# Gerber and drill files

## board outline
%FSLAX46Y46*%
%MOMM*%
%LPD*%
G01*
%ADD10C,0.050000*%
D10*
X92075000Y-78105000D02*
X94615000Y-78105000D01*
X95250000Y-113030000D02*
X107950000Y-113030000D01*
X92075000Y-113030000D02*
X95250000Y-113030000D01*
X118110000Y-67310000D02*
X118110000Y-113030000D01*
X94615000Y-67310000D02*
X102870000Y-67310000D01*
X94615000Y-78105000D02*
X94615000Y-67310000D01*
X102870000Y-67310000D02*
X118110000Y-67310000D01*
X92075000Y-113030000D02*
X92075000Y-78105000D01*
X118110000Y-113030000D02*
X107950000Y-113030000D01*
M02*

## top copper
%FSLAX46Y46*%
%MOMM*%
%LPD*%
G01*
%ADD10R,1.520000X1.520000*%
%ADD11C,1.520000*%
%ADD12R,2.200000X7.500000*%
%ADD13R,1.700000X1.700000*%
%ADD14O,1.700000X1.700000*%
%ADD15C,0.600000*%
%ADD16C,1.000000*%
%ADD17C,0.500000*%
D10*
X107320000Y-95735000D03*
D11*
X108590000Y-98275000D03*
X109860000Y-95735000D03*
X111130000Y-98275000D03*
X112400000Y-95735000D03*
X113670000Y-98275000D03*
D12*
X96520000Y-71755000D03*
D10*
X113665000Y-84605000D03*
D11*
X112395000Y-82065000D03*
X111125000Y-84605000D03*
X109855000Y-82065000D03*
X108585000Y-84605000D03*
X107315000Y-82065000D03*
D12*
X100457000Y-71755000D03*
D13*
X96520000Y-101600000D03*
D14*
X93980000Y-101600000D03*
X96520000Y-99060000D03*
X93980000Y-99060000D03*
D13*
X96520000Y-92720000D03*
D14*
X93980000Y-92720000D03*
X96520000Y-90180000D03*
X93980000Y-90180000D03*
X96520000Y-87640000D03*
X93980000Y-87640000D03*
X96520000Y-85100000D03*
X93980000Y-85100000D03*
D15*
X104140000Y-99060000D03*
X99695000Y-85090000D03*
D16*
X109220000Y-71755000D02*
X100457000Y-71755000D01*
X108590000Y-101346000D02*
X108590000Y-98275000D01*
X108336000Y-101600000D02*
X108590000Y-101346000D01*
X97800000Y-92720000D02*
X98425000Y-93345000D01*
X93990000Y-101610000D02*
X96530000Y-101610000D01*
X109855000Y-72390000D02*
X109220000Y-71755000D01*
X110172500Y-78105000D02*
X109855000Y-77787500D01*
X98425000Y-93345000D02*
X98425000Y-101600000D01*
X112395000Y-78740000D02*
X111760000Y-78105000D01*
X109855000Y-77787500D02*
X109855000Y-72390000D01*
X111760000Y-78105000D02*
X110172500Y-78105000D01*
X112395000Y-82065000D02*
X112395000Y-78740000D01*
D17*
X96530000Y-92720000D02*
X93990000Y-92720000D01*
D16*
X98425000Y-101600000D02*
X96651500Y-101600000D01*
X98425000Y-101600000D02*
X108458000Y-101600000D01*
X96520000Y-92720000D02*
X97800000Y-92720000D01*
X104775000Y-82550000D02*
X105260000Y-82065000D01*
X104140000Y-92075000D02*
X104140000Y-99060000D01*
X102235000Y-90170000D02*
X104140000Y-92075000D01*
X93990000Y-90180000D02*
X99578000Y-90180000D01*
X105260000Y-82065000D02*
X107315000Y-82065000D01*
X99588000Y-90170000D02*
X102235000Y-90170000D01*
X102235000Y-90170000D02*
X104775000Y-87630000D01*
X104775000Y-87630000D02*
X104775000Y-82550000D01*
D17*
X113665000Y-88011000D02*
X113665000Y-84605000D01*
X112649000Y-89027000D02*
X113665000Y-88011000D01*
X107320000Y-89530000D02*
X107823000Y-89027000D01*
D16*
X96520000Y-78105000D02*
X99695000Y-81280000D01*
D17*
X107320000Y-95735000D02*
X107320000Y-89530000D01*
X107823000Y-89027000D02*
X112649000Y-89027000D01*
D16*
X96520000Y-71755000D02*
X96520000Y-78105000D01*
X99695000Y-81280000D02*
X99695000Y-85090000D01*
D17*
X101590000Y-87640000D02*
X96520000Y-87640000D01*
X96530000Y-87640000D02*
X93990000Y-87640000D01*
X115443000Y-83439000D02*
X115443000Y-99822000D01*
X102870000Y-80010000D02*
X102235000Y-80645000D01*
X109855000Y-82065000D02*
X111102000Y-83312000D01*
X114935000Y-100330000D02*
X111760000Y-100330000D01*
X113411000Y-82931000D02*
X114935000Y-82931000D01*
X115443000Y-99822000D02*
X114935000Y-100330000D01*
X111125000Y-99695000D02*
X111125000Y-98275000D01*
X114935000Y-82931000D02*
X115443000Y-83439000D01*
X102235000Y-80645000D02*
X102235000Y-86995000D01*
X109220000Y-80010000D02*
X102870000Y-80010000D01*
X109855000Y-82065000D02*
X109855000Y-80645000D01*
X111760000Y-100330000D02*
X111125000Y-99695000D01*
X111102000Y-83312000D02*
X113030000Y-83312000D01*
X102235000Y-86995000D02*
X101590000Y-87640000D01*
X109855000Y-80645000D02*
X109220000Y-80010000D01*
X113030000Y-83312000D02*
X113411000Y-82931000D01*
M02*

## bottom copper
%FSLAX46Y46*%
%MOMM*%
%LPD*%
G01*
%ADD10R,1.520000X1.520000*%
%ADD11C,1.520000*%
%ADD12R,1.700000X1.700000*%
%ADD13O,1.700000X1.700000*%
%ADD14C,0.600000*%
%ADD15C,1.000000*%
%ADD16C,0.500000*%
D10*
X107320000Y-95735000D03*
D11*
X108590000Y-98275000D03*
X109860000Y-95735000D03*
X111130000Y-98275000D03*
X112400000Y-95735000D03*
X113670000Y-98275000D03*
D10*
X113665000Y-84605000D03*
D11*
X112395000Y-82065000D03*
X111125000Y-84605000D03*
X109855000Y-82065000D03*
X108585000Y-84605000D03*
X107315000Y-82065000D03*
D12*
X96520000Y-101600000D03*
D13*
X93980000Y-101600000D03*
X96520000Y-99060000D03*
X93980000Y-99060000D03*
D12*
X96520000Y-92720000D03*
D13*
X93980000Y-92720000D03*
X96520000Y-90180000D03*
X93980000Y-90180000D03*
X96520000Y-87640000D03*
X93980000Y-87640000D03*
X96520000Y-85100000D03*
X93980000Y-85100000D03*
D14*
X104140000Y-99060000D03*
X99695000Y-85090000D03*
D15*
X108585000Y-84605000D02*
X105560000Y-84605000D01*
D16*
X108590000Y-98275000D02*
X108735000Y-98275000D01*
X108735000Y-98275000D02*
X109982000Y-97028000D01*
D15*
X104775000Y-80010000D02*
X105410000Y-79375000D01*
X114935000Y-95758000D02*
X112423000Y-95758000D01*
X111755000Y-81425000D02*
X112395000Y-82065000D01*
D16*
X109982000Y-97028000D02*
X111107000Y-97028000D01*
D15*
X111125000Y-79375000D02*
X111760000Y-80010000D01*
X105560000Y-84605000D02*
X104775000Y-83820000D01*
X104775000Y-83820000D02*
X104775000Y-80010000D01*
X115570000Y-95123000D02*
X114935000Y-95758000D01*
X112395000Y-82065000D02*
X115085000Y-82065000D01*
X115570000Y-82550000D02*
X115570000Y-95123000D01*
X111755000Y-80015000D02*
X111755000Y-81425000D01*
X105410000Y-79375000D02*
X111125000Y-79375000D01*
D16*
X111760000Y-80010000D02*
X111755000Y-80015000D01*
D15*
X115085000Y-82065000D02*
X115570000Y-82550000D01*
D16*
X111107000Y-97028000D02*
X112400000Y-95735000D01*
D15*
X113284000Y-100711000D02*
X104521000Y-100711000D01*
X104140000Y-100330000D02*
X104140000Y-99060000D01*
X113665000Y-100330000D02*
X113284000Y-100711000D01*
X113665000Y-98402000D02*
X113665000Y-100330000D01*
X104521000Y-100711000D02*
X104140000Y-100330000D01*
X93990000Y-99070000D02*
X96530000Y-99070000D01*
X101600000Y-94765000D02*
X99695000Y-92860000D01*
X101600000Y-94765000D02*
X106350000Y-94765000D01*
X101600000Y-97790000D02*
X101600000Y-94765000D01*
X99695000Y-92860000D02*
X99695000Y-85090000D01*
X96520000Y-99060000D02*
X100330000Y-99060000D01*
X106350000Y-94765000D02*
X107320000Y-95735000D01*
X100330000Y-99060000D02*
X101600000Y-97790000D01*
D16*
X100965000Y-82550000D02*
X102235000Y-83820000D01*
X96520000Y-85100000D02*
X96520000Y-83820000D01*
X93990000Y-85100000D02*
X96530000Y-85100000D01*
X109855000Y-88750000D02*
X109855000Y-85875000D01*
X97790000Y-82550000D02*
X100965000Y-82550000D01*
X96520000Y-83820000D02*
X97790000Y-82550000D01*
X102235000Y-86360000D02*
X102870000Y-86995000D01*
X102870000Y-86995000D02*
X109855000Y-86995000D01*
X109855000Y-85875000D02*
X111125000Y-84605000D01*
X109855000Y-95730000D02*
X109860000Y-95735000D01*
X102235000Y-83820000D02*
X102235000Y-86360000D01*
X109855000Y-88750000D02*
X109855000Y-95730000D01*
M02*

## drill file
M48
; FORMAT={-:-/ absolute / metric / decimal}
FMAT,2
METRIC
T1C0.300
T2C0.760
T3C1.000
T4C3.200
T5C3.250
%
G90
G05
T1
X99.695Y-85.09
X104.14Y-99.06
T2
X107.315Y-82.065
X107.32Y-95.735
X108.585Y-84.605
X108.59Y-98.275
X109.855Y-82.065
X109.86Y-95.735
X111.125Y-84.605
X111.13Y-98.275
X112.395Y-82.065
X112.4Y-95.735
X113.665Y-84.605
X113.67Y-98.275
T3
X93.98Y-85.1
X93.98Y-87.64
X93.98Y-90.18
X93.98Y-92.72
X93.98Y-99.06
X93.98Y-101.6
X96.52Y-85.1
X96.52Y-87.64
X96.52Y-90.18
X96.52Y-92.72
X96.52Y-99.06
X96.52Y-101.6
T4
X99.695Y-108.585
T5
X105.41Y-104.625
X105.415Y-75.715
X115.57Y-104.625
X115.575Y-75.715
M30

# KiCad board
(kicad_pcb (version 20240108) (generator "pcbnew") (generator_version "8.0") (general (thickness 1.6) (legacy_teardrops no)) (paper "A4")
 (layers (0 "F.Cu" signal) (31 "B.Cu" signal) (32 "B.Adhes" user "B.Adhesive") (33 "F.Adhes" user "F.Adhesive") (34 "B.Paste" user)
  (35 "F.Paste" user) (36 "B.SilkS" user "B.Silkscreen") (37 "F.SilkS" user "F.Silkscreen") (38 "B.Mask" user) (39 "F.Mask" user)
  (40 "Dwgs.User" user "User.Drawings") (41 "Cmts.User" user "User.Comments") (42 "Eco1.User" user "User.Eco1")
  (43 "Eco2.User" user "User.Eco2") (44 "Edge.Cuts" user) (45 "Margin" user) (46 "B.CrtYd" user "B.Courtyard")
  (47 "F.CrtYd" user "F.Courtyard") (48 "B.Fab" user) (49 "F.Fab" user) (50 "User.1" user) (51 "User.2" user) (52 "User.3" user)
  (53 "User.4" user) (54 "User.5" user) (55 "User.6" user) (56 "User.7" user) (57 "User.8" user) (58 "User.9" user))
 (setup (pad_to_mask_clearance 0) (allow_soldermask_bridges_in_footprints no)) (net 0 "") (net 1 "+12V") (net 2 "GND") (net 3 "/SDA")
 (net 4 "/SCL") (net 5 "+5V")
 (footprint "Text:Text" (layer "F.Cu") (at 106.68 116.84)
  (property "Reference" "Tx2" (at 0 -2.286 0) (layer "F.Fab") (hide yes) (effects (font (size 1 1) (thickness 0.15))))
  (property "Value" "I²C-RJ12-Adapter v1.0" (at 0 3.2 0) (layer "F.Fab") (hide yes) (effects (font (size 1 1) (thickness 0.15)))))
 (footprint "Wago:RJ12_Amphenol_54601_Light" (layer "F.Cu") (at 107.32 95.735)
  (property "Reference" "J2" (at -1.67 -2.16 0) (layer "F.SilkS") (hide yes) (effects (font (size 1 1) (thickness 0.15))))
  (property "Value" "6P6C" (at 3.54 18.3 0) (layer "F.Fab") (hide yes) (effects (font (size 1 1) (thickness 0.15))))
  (pad "" np_thru_hole circle (at -1.91 8.89) (size 3.25 3.25) (drill 3.25) (layers "*.Cu" "*.Mask"))
  (pad "" np_thru_hole circle (at 8.25 8.89) (size 3.25 3.25) (drill 3.25) (layers "*.Cu" "*.Mask"))
  (pad "1" thru_hole rect (at 0 0) (size 1.52 1.52) (drill 0.76) (layers "*.Cu" "*.Mask") (remove_unused_layers no) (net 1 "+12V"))
  (pad "2" thru_hole circle (at 1.27 2.54) (size 1.52 1.52) (drill 0.76) (layers "*.Cu" "*.Mask") (remove_unused_layers no) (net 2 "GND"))
  (pad "3" thru_hole circle (at 2.54 0) (size 1.52 1.52) (drill 0.76) (layers "*.Cu" "*.Mask") (remove_unused_layers no) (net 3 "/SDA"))
  (pad "4" thru_hole circle (at 3.81 2.54) (size 1.52 1.52) (drill 0.76) (layers "*.Cu" "*.Mask") (remove_unused_layers no) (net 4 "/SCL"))
  (pad "5" thru_hole circle (at 5.08 0) (size 1.52 1.52) (drill 0.76) (layers "*.Cu" "*.Mask") (remove_unused_layers no) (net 2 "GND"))
  (pad "6" thru_hole circle (at 6.35 2.54) (size 1.52 1.52) (drill 0.76) (layers "*.Cu" "*.Mask") (remove_unused_layers no) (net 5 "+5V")))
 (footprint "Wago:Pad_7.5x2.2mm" (layer "F.Cu") (at 96.52 71.755 90)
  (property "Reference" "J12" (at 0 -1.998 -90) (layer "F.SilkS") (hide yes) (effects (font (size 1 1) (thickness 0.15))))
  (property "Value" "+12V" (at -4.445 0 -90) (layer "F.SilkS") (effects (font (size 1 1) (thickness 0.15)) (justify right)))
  (pad "1" smd rect (at 0 0 90) (size 7.5 2.2) (layers "F.Cu" "F.Mask") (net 1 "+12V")))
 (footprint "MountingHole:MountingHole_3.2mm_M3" (layer "F.Cu") (at 99.695 108.585)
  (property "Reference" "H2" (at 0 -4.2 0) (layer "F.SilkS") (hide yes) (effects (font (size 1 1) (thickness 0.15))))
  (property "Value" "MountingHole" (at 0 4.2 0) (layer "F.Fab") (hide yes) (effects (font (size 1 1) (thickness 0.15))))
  (pad "" np_thru_hole circle (at 0 0) (size 3.2 3.2) (drill 3.2) (layers "F&B.Cu" "*.Mask")))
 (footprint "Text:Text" (layer "F.Cu") (at 81.28 95.25 90)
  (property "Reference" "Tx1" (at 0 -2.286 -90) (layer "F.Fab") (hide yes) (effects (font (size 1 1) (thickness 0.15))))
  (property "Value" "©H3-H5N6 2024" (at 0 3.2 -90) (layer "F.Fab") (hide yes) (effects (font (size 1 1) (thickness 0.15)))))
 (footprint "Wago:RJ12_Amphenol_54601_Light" (layer "F.Cu") (at 113.665 84.605 180)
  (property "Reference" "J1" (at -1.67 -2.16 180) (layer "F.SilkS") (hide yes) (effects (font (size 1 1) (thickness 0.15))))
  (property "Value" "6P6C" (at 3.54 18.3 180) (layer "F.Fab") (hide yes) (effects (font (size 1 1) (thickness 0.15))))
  (pad "" np_thru_hole circle (at -1.91 8.89 180) (size 3.25 3.25) (drill 3.25) (layers "*.Cu" "*.Mask"))
  (pad "" np_thru_hole circle (at 8.25 8.89 180) (size 3.25 3.25) (drill 3.25) (layers "*.Cu" "*.Mask"))
  (pad "1" thru_hole rect (at 0 0 180) (size 1.52 1.52) (drill 0.76) (layers "*.Cu" "*.Mask") (remove_unused_layers no) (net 1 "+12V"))
  (pad "2" thru_hole circle (at 1.27 2.54 180) (size 1.52 1.52) (drill 0.76) (layers "*.Cu" "*.Mask") (remove_unused_layers no)
   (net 2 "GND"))
  (pad "3" thru_hole circle (at 2.54 0 180) (size 1.52 1.52) (drill 0.76) (layers "*.Cu" "*.Mask") (remove_unused_layers no) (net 3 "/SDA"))
  (pad "4" thru_hole circle (at 3.81 2.54 180) (size 1.52 1.52) (drill 0.76) (layers "*.Cu" "*.Mask") (remove_unused_layers no)
   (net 4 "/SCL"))
  (pad "5" thru_hole circle (at 5.08 0 180) (size 1.52 1.52) (drill 0.76) (layers "*.Cu" "*.Mask") (remove_unused_layers no) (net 2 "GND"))
  (pad "6" thru_hole circle (at 6.35 2.54 180) (size 1.52 1.52) (drill 0.76) (layers "*.Cu" "*.Mask") (remove_unused_layers no)
   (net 5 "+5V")))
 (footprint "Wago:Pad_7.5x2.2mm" (layer "F.Cu") (at 100.457 71.755 90)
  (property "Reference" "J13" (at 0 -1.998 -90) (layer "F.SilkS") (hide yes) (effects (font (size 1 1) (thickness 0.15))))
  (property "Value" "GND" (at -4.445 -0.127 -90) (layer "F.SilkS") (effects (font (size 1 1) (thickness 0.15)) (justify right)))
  (pad "1" smd rect (at 0 0 90) (size 7.5 2.2) (layers "F.Cu" "F.Mask") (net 2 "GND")))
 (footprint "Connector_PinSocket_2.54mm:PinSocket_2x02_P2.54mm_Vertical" (layer "B.Cu") (at 96.52 101.6)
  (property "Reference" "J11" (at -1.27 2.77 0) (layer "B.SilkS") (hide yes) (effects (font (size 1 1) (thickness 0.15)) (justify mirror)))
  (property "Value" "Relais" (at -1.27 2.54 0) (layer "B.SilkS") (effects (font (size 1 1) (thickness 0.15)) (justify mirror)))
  (pad "1" thru_hole rect (at 0 0) (size 1.7 1.7) (drill 1) (layers "*.Cu" "*.Mask") (remove_unused_layers no) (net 2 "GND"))
  (pad "2" thru_hole oval (at -2.54 0) (size 1.7 1.7) (drill 1) (layers "*.Cu" "*.Mask") (remove_unused_layers no) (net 2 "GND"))
  (pad "3" thru_hole oval (at 0 -2.54) (size 1.7 1.7) (drill 1) (layers "*.Cu" "*.Mask") (remove_unused_layers no) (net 1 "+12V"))
  (pad "4" thru_hole oval (at -2.54 -2.54) (size 1.7 1.7) (drill 1) (layers "*.Cu" "*.Mask") (remove_unused_layers no) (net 1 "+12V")))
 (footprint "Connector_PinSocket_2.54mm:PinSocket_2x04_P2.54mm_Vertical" (layer "B.Cu") (at 96.52 92.72)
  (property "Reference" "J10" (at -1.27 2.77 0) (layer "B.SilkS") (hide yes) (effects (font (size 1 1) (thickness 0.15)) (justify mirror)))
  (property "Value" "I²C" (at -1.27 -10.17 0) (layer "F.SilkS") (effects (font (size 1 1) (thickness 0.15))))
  (pad "1" thru_hole rect (at 0 0) (size 1.7 1.7) (drill 1) (layers "*.Cu" "*.Mask") (remove_unused_layers no) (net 2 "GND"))
  (pad "2" thru_hole oval (at -2.54 0) (size 1.7 1.7) (drill 1) (layers "*.Cu" "*.Mask") (remove_unused_layers no) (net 2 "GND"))
  (pad "3" thru_hole oval (at 0 -2.54) (size 1.7 1.7) (drill 1) (layers "*.Cu" "*.Mask") (remove_unused_layers no) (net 5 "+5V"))
  (pad "4" thru_hole oval (at -2.54 -2.54) (size 1.7 1.7) (drill 1) (layers "*.Cu" "*.Mask") (remove_unused_layers no) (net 5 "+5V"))
  (pad "5" thru_hole oval (at 0 -5.08) (size 1.7 1.7) (drill 1) (layers "*.Cu" "*.Mask") (remove_unused_layers no) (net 4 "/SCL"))
  (pad "6" thru_hole oval (at -2.54 -5.08) (size 1.7 1.7) (drill 1) (layers "*.Cu" "*.Mask") (remove_unused_layers no) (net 4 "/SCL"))
  (pad "7" thru_hole oval (at 0 -7.62) (size 1.7 1.7) (drill 1) (layers "*.Cu" "*.Mask") (remove_unused_layers no) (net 3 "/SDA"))
  (pad "8" thru_hole oval (at -2.54 -7.62) (size 1.7 1.7) (drill 1) (layers "*.Cu" "*.Mask") (remove_unused_layers no) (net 3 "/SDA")))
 (gr_line (start 92.075 78.105) (end 94.615 78.105) (stroke (width 0.05) (type default)) (layer "Edge.Cuts"))
 (gr_line (start 95.25 113.03) (end 107.95 113.03) (stroke (width 0.05) (type default)) (layer "Edge.Cuts"))
 (gr_line (start 92.075 113.03) (end 95.25 113.03) (stroke (width 0.05) (type default)) (layer "Edge.Cuts"))
 (gr_line (start 118.11 67.31) (end 118.11 113.03) (stroke (width 0.05) (type default)) (layer "Edge.Cuts"))
 (gr_line (start 94.615 67.31) (end 102.87 67.31) (stroke (width 0.05) (type default)) (layer "Edge.Cuts"))
 (gr_line (start 94.615 78.105) (end 94.615 67.31) (stroke (width 0.05) (type default)) (layer "Edge.Cuts"))
 (gr_line (start 102.87 67.31) (end 118.11 67.31) (stroke (width 0.05) (type default)) (layer "Edge.Cuts"))
 (gr_line (start 92.075 113.03) (end 92.075 78.105) (stroke (width 0.05) (type default)) (layer "Edge.Cuts"))
 (gr_line (start 118.11 113.03) (end 107.95 113.03) (stroke (width 0.05) (type default)) (layer "Edge.Cuts"))
 (segment (start 109.22 71.755) (end 100.457 71.755) (width 1) (layer "F.Cu") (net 2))
 (segment (start 108.59 101.346) (end 108.59 98.275) (width 1) (layer "F.Cu") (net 2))
 (segment (start 108.336 101.6) (end 108.59 101.346) (width 1) (layer "F.Cu") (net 2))
 (segment (start 97.8 92.72) (end 98.425 93.345) (width 1) (layer "F.Cu") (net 2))
 (segment (start 93.99 101.61) (end 96.53 101.61) (width 1) (layer "F.Cu") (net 2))
 (segment (start 109.855 72.39) (end 109.22 71.755) (width 1) (layer "F.Cu") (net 2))
 (segment (start 110.1725 78.105) (end 109.855 77.7875) (width 1) (layer "F.Cu") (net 2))
 (segment (start 98.425 93.345) (end 98.425 101.6) (width 1) (layer "F.Cu") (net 2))
 (segment (start 112.395 78.74) (end 111.76 78.105) (width 1) (layer "F.Cu") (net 2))
 (segment (start 109.855 77.7875) (end 109.855 72.39) (width 1) (layer "F.Cu") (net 2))
 (segment (start 111.76 78.105) (end 110.1725 78.105) (width 1) (layer "F.Cu") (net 2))
 (segment (start 112.395 82.065) (end 112.395 78.74) (width 1) (layer "F.Cu") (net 2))
 (segment (start 96.53 92.72) (end 93.99 92.72) (width 0.5) (layer "F.Cu") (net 2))
 (segment (start 98.425 101.6) (end 96.6515 101.6) (width 1) (layer "F.Cu") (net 2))
 (segment (start 98.425 101.6) (end 108.458 101.6) (width 1) (layer "F.Cu") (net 2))
 (segment (start 96.52 92.72) (end 97.8 92.72) (width 1) (layer "F.Cu") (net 2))
 (segment (start 108.585 84.605) (end 105.56 84.605) (width 1) (layer "B.Cu") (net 2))
 (segment (start 108.59 98.275) (end 108.735 98.275) (width 0.5) (layer "B.Cu") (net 2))
 (segment (start 108.735 98.275) (end 109.982 97.028) (width 0.5) (layer "B.Cu") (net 2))
 (segment (start 104.775 80.01) (end 105.41 79.375) (width 1) (layer "B.Cu") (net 2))
 (segment (start 114.935 95.758) (end 112.423 95.758) (width 1) (layer "B.Cu") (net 2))
 (segment (start 111.755 81.425) (end 112.395 82.065) (width 1) (layer "B.Cu") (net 2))
 (segment (start 109.982 97.028) (end 111.107 97.028) (width 0.5) (layer "B.Cu") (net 2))
 (segment (start 111.125 79.375) (end 111.76 80.01) (width 1) (layer "B.Cu") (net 2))
 (segment (start 105.56 84.605) (end 104.775 83.82) (width 1) (layer "B.Cu") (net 2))
 (segment (start 104.775 83.82) (end 104.775 80.01) (width 1) (layer "B.Cu") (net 2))
 (segment (start 115.57 95.123) (end 114.935 95.758) (width 1) (layer "B.Cu") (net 2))
 (segment (start 112.395 82.065) (end 115.085 82.065) (width 1) (layer "B.Cu") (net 2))
 (segment (start 115.57 82.55) (end 115.57 95.123) (width 1) (layer "B.Cu") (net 2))
 (segment (start 111.755 80.015) (end 111.755 81.425) (width 1) (layer "B.Cu") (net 2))
 (segment (start 105.41 79.375) (end 111.125 79.375) (width 1) (layer "B.Cu") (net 2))
 (segment (start 111.76 80.01) (end 111.755 80.015) (width 0.5) (layer "B.Cu") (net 2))
 (segment (start 115.085 82.065) (end 115.57 82.55) (width 1) (layer "B.Cu") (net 2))
 (segment (start 111.107 97.028) (end 112.4 95.735) (width 0.5) (layer "B.Cu") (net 2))
 (segment (start 104.775 82.55) (end 105.26 82.065) (width 1) (layer "F.Cu") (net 5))
 (segment (start 104.14 92.075) (end 104.14 99.06) (width 1) (layer "F.Cu") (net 5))
 (segment (start 102.235 90.17) (end 104.14 92.075) (width 1) (layer "F.Cu") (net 5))
 (segment (start 93.99 90.18) (end 99.578 90.18) (width 1) (layer "F.Cu") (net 5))
 (segment (start 105.26 82.065) (end 107.315 82.065) (width 1) (layer "F.Cu") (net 5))
 (segment (start 99.588 90.17) (end 102.235 90.17) (width 1) (layer "F.Cu") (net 5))
 (segment (start 102.235 90.17) (end 104.775 87.63) (width 1) (layer "F.Cu") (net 5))
 (segment (start 104.775 87.63) (end 104.775 82.55) (width 1) (layer "F.Cu") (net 5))
 (via (at 104.14 99.06) (size 0.6) (drill 0.3) (layers "F.Cu" "B.Cu") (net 5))
 (segment (start 113.284 100.711) (end 104.521 100.711) (width 1) (layer "B.Cu") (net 5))
 (segment (start 104.14 100.33) (end 104.14 99.06) (width 1) (layer "B.Cu") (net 5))
 (segment (start 113.665 100.33) (end 113.284 100.711) (width 1) (layer "B.Cu") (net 5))
 (segment (start 113.665 98.402) (end 113.665 100.33) (width 1) (layer "B.Cu") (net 5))
 (segment (start 104.521 100.711) (end 104.14 100.33) (width 1) (layer "B.Cu") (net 5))
 (segment (start 113.665 88.011) (end 113.665 84.605) (width 0.5) (layer "F.Cu") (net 1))
 (segment (start 112.649 89.027) (end 113.665 88.011) (width 0.5) (layer "F.Cu") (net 1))
 (segment (start 107.32 89.53) (end 107.823 89.027) (width 0.5) (layer "F.Cu") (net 1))
 (segment (start 96.52 78.105) (end 99.695 81.28) (width 1) (layer "F.Cu") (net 1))
 (segment (start 107.32 95.735) (end 107.32 89.53) (width 0.5) (layer "F.Cu") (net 1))
 (segment (start 107.823 89.027) (end 112.649 89.027) (width 0.5) (layer "F.Cu") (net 1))
 (segment (start 96.52 71.755) (end 96.52 78.105) (width 1) (layer "F.Cu") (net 1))
 (segment (start 99.695 81.28) (end 99.695 85.09) (width 1) (layer "F.Cu") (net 1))
 (via (at 99.695 85.09) (size 0.6) (drill 0.3) (layers "F.Cu" "B.Cu") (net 1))
 (segment (start 93.99 99.07) (end 96.53 99.07) (width 1) (layer "B.Cu") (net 1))
 (segment (start 101.6 94.765) (end 99.695 92.86) (width 1) (layer "B.Cu") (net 1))
 (segment (start 101.6 94.765) (end 106.35 94.765) (width 1) (layer "B.Cu") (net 1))
 (segment (start 101.6 97.79) (end 101.6 94.765) (width 1) (layer "B.Cu") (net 1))
 (segment (start 99.695 92.86) (end 99.695 85.09) (width 1) (layer "B.Cu") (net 1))
 (segment (start 96.52 99.06) (end 100.33 99.06) (width 1) (layer "B.Cu") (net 1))
 (segment (start 106.35 94.765) (end 107.32 95.735) (width 1) (layer "B.Cu") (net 1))
 (segment (start 100.33 99.06) (end 101.6 97.79) (width 1) (layer "B.Cu") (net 1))
 (segment (start 100.965 82.55) (end 102.235 83.82) (width 0.5) (layer "B.Cu") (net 3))
 (segment (start 96.52 85.1) (end 96.52 83.82) (width 0.5) (layer "B.Cu") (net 3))
 (segment (start 93.99 85.1) (end 96.53 85.1) (width 0.5) (layer "B.Cu") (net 3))
 (segment (start 109.855 88.75) (end 109.855 85.875) (width 0.5) (layer "B.Cu") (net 3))
 (segment (start 97.79 82.55) (end 100.965 82.55) (width 0.5) (layer "B.Cu") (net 3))
 (segment (start 96.52 83.82) (end 97.79 82.55) (width 0.5) (layer "B.Cu") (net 3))
 (segment (start 102.235 86.36) (end 102.87 86.995) (width 0.5) (layer "B.Cu") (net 3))
 (segment (start 102.87 86.995) (end 109.855 86.995) (width 0.5) (layer "B.Cu") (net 3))
 (segment (start 109.855 85.875) (end 111.125 84.605) (width 0.5) (layer "B.Cu") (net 3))
 (segment (start 109.855 95.73) (end 109.86 95.735) (width 0.5) (layer "B.Cu") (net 3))
 (segment (start 102.235 83.82) (end 102.235 86.36) (width 0.5) (layer "B.Cu") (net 3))
 (segment (start 109.855 88.75) (end 109.855 95.73) (width 0.5) (layer "B.Cu") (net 3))
 (segment (start 101.59 87.64) (end 96.52 87.64) (width 0.5) (layer "F.Cu") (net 4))
 (segment (start 96.53 87.64) (end 93.99 87.64) (width 0.5) (layer "F.Cu") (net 4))
 (segment (start 115.443 83.439) (end 115.443 99.822) (width 0.5) (layer "F.Cu") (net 4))
 (segment (start 102.87 80.01) (end 102.235 80.645) (width 0.5) (layer "F.Cu") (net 4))
 (segment (start 109.855 82.065) (end 111.102 83.312) (width 0.5) (layer "F.Cu") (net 4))
 (segment (start 114.935 100.33) (end 111.76 100.33) (width 0.5) (layer "F.Cu") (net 4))
 (segment (start 113.411 82.931) (end 114.935 82.931) (width 0.5) (layer "F.Cu") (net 4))
 (segment (start 115.443 99.822) (end 114.935 100.33) (width 0.5) (layer "F.Cu") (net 4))
 (segment (start 111.125 99.695) (end 111.125 98.275) (width 0.5) (layer "F.Cu") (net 4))
 (segment (start 114.935 82.931) (end 115.443 83.439) (width 0.5) (layer "F.Cu") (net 4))
 (segment (start 102.235 80.645) (end 102.235 86.995) (width 0.5) (layer "F.Cu") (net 4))
 (segment (start 109.22 80.01) (end 102.87 80.01) (width 0.5) (layer "F.Cu") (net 4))
 (segment (start 109.855 82.065) (end 109.855 80.645) (width 0.5) (layer "F.Cu") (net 4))
 (segment (start 111.76 100.33) (end 111.125 99.695) (width 0.5) (layer "F.Cu") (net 4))
 (segment (start 111.102 83.312) (end 113.03 83.312) (width 0.5) (layer "F.Cu") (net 4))
 (segment (start 102.235 86.995) (end 101.59 87.64) (width 0.5) (layer "F.Cu") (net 4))
 (segment (start 109.855 80.645) (end 109.22 80.01) (width 0.5) (layer "F.Cu") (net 4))
 (segment (start 113.03 83.312) (end 113.411 82.931) (width 0.5) (layer "F.Cu") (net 4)))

